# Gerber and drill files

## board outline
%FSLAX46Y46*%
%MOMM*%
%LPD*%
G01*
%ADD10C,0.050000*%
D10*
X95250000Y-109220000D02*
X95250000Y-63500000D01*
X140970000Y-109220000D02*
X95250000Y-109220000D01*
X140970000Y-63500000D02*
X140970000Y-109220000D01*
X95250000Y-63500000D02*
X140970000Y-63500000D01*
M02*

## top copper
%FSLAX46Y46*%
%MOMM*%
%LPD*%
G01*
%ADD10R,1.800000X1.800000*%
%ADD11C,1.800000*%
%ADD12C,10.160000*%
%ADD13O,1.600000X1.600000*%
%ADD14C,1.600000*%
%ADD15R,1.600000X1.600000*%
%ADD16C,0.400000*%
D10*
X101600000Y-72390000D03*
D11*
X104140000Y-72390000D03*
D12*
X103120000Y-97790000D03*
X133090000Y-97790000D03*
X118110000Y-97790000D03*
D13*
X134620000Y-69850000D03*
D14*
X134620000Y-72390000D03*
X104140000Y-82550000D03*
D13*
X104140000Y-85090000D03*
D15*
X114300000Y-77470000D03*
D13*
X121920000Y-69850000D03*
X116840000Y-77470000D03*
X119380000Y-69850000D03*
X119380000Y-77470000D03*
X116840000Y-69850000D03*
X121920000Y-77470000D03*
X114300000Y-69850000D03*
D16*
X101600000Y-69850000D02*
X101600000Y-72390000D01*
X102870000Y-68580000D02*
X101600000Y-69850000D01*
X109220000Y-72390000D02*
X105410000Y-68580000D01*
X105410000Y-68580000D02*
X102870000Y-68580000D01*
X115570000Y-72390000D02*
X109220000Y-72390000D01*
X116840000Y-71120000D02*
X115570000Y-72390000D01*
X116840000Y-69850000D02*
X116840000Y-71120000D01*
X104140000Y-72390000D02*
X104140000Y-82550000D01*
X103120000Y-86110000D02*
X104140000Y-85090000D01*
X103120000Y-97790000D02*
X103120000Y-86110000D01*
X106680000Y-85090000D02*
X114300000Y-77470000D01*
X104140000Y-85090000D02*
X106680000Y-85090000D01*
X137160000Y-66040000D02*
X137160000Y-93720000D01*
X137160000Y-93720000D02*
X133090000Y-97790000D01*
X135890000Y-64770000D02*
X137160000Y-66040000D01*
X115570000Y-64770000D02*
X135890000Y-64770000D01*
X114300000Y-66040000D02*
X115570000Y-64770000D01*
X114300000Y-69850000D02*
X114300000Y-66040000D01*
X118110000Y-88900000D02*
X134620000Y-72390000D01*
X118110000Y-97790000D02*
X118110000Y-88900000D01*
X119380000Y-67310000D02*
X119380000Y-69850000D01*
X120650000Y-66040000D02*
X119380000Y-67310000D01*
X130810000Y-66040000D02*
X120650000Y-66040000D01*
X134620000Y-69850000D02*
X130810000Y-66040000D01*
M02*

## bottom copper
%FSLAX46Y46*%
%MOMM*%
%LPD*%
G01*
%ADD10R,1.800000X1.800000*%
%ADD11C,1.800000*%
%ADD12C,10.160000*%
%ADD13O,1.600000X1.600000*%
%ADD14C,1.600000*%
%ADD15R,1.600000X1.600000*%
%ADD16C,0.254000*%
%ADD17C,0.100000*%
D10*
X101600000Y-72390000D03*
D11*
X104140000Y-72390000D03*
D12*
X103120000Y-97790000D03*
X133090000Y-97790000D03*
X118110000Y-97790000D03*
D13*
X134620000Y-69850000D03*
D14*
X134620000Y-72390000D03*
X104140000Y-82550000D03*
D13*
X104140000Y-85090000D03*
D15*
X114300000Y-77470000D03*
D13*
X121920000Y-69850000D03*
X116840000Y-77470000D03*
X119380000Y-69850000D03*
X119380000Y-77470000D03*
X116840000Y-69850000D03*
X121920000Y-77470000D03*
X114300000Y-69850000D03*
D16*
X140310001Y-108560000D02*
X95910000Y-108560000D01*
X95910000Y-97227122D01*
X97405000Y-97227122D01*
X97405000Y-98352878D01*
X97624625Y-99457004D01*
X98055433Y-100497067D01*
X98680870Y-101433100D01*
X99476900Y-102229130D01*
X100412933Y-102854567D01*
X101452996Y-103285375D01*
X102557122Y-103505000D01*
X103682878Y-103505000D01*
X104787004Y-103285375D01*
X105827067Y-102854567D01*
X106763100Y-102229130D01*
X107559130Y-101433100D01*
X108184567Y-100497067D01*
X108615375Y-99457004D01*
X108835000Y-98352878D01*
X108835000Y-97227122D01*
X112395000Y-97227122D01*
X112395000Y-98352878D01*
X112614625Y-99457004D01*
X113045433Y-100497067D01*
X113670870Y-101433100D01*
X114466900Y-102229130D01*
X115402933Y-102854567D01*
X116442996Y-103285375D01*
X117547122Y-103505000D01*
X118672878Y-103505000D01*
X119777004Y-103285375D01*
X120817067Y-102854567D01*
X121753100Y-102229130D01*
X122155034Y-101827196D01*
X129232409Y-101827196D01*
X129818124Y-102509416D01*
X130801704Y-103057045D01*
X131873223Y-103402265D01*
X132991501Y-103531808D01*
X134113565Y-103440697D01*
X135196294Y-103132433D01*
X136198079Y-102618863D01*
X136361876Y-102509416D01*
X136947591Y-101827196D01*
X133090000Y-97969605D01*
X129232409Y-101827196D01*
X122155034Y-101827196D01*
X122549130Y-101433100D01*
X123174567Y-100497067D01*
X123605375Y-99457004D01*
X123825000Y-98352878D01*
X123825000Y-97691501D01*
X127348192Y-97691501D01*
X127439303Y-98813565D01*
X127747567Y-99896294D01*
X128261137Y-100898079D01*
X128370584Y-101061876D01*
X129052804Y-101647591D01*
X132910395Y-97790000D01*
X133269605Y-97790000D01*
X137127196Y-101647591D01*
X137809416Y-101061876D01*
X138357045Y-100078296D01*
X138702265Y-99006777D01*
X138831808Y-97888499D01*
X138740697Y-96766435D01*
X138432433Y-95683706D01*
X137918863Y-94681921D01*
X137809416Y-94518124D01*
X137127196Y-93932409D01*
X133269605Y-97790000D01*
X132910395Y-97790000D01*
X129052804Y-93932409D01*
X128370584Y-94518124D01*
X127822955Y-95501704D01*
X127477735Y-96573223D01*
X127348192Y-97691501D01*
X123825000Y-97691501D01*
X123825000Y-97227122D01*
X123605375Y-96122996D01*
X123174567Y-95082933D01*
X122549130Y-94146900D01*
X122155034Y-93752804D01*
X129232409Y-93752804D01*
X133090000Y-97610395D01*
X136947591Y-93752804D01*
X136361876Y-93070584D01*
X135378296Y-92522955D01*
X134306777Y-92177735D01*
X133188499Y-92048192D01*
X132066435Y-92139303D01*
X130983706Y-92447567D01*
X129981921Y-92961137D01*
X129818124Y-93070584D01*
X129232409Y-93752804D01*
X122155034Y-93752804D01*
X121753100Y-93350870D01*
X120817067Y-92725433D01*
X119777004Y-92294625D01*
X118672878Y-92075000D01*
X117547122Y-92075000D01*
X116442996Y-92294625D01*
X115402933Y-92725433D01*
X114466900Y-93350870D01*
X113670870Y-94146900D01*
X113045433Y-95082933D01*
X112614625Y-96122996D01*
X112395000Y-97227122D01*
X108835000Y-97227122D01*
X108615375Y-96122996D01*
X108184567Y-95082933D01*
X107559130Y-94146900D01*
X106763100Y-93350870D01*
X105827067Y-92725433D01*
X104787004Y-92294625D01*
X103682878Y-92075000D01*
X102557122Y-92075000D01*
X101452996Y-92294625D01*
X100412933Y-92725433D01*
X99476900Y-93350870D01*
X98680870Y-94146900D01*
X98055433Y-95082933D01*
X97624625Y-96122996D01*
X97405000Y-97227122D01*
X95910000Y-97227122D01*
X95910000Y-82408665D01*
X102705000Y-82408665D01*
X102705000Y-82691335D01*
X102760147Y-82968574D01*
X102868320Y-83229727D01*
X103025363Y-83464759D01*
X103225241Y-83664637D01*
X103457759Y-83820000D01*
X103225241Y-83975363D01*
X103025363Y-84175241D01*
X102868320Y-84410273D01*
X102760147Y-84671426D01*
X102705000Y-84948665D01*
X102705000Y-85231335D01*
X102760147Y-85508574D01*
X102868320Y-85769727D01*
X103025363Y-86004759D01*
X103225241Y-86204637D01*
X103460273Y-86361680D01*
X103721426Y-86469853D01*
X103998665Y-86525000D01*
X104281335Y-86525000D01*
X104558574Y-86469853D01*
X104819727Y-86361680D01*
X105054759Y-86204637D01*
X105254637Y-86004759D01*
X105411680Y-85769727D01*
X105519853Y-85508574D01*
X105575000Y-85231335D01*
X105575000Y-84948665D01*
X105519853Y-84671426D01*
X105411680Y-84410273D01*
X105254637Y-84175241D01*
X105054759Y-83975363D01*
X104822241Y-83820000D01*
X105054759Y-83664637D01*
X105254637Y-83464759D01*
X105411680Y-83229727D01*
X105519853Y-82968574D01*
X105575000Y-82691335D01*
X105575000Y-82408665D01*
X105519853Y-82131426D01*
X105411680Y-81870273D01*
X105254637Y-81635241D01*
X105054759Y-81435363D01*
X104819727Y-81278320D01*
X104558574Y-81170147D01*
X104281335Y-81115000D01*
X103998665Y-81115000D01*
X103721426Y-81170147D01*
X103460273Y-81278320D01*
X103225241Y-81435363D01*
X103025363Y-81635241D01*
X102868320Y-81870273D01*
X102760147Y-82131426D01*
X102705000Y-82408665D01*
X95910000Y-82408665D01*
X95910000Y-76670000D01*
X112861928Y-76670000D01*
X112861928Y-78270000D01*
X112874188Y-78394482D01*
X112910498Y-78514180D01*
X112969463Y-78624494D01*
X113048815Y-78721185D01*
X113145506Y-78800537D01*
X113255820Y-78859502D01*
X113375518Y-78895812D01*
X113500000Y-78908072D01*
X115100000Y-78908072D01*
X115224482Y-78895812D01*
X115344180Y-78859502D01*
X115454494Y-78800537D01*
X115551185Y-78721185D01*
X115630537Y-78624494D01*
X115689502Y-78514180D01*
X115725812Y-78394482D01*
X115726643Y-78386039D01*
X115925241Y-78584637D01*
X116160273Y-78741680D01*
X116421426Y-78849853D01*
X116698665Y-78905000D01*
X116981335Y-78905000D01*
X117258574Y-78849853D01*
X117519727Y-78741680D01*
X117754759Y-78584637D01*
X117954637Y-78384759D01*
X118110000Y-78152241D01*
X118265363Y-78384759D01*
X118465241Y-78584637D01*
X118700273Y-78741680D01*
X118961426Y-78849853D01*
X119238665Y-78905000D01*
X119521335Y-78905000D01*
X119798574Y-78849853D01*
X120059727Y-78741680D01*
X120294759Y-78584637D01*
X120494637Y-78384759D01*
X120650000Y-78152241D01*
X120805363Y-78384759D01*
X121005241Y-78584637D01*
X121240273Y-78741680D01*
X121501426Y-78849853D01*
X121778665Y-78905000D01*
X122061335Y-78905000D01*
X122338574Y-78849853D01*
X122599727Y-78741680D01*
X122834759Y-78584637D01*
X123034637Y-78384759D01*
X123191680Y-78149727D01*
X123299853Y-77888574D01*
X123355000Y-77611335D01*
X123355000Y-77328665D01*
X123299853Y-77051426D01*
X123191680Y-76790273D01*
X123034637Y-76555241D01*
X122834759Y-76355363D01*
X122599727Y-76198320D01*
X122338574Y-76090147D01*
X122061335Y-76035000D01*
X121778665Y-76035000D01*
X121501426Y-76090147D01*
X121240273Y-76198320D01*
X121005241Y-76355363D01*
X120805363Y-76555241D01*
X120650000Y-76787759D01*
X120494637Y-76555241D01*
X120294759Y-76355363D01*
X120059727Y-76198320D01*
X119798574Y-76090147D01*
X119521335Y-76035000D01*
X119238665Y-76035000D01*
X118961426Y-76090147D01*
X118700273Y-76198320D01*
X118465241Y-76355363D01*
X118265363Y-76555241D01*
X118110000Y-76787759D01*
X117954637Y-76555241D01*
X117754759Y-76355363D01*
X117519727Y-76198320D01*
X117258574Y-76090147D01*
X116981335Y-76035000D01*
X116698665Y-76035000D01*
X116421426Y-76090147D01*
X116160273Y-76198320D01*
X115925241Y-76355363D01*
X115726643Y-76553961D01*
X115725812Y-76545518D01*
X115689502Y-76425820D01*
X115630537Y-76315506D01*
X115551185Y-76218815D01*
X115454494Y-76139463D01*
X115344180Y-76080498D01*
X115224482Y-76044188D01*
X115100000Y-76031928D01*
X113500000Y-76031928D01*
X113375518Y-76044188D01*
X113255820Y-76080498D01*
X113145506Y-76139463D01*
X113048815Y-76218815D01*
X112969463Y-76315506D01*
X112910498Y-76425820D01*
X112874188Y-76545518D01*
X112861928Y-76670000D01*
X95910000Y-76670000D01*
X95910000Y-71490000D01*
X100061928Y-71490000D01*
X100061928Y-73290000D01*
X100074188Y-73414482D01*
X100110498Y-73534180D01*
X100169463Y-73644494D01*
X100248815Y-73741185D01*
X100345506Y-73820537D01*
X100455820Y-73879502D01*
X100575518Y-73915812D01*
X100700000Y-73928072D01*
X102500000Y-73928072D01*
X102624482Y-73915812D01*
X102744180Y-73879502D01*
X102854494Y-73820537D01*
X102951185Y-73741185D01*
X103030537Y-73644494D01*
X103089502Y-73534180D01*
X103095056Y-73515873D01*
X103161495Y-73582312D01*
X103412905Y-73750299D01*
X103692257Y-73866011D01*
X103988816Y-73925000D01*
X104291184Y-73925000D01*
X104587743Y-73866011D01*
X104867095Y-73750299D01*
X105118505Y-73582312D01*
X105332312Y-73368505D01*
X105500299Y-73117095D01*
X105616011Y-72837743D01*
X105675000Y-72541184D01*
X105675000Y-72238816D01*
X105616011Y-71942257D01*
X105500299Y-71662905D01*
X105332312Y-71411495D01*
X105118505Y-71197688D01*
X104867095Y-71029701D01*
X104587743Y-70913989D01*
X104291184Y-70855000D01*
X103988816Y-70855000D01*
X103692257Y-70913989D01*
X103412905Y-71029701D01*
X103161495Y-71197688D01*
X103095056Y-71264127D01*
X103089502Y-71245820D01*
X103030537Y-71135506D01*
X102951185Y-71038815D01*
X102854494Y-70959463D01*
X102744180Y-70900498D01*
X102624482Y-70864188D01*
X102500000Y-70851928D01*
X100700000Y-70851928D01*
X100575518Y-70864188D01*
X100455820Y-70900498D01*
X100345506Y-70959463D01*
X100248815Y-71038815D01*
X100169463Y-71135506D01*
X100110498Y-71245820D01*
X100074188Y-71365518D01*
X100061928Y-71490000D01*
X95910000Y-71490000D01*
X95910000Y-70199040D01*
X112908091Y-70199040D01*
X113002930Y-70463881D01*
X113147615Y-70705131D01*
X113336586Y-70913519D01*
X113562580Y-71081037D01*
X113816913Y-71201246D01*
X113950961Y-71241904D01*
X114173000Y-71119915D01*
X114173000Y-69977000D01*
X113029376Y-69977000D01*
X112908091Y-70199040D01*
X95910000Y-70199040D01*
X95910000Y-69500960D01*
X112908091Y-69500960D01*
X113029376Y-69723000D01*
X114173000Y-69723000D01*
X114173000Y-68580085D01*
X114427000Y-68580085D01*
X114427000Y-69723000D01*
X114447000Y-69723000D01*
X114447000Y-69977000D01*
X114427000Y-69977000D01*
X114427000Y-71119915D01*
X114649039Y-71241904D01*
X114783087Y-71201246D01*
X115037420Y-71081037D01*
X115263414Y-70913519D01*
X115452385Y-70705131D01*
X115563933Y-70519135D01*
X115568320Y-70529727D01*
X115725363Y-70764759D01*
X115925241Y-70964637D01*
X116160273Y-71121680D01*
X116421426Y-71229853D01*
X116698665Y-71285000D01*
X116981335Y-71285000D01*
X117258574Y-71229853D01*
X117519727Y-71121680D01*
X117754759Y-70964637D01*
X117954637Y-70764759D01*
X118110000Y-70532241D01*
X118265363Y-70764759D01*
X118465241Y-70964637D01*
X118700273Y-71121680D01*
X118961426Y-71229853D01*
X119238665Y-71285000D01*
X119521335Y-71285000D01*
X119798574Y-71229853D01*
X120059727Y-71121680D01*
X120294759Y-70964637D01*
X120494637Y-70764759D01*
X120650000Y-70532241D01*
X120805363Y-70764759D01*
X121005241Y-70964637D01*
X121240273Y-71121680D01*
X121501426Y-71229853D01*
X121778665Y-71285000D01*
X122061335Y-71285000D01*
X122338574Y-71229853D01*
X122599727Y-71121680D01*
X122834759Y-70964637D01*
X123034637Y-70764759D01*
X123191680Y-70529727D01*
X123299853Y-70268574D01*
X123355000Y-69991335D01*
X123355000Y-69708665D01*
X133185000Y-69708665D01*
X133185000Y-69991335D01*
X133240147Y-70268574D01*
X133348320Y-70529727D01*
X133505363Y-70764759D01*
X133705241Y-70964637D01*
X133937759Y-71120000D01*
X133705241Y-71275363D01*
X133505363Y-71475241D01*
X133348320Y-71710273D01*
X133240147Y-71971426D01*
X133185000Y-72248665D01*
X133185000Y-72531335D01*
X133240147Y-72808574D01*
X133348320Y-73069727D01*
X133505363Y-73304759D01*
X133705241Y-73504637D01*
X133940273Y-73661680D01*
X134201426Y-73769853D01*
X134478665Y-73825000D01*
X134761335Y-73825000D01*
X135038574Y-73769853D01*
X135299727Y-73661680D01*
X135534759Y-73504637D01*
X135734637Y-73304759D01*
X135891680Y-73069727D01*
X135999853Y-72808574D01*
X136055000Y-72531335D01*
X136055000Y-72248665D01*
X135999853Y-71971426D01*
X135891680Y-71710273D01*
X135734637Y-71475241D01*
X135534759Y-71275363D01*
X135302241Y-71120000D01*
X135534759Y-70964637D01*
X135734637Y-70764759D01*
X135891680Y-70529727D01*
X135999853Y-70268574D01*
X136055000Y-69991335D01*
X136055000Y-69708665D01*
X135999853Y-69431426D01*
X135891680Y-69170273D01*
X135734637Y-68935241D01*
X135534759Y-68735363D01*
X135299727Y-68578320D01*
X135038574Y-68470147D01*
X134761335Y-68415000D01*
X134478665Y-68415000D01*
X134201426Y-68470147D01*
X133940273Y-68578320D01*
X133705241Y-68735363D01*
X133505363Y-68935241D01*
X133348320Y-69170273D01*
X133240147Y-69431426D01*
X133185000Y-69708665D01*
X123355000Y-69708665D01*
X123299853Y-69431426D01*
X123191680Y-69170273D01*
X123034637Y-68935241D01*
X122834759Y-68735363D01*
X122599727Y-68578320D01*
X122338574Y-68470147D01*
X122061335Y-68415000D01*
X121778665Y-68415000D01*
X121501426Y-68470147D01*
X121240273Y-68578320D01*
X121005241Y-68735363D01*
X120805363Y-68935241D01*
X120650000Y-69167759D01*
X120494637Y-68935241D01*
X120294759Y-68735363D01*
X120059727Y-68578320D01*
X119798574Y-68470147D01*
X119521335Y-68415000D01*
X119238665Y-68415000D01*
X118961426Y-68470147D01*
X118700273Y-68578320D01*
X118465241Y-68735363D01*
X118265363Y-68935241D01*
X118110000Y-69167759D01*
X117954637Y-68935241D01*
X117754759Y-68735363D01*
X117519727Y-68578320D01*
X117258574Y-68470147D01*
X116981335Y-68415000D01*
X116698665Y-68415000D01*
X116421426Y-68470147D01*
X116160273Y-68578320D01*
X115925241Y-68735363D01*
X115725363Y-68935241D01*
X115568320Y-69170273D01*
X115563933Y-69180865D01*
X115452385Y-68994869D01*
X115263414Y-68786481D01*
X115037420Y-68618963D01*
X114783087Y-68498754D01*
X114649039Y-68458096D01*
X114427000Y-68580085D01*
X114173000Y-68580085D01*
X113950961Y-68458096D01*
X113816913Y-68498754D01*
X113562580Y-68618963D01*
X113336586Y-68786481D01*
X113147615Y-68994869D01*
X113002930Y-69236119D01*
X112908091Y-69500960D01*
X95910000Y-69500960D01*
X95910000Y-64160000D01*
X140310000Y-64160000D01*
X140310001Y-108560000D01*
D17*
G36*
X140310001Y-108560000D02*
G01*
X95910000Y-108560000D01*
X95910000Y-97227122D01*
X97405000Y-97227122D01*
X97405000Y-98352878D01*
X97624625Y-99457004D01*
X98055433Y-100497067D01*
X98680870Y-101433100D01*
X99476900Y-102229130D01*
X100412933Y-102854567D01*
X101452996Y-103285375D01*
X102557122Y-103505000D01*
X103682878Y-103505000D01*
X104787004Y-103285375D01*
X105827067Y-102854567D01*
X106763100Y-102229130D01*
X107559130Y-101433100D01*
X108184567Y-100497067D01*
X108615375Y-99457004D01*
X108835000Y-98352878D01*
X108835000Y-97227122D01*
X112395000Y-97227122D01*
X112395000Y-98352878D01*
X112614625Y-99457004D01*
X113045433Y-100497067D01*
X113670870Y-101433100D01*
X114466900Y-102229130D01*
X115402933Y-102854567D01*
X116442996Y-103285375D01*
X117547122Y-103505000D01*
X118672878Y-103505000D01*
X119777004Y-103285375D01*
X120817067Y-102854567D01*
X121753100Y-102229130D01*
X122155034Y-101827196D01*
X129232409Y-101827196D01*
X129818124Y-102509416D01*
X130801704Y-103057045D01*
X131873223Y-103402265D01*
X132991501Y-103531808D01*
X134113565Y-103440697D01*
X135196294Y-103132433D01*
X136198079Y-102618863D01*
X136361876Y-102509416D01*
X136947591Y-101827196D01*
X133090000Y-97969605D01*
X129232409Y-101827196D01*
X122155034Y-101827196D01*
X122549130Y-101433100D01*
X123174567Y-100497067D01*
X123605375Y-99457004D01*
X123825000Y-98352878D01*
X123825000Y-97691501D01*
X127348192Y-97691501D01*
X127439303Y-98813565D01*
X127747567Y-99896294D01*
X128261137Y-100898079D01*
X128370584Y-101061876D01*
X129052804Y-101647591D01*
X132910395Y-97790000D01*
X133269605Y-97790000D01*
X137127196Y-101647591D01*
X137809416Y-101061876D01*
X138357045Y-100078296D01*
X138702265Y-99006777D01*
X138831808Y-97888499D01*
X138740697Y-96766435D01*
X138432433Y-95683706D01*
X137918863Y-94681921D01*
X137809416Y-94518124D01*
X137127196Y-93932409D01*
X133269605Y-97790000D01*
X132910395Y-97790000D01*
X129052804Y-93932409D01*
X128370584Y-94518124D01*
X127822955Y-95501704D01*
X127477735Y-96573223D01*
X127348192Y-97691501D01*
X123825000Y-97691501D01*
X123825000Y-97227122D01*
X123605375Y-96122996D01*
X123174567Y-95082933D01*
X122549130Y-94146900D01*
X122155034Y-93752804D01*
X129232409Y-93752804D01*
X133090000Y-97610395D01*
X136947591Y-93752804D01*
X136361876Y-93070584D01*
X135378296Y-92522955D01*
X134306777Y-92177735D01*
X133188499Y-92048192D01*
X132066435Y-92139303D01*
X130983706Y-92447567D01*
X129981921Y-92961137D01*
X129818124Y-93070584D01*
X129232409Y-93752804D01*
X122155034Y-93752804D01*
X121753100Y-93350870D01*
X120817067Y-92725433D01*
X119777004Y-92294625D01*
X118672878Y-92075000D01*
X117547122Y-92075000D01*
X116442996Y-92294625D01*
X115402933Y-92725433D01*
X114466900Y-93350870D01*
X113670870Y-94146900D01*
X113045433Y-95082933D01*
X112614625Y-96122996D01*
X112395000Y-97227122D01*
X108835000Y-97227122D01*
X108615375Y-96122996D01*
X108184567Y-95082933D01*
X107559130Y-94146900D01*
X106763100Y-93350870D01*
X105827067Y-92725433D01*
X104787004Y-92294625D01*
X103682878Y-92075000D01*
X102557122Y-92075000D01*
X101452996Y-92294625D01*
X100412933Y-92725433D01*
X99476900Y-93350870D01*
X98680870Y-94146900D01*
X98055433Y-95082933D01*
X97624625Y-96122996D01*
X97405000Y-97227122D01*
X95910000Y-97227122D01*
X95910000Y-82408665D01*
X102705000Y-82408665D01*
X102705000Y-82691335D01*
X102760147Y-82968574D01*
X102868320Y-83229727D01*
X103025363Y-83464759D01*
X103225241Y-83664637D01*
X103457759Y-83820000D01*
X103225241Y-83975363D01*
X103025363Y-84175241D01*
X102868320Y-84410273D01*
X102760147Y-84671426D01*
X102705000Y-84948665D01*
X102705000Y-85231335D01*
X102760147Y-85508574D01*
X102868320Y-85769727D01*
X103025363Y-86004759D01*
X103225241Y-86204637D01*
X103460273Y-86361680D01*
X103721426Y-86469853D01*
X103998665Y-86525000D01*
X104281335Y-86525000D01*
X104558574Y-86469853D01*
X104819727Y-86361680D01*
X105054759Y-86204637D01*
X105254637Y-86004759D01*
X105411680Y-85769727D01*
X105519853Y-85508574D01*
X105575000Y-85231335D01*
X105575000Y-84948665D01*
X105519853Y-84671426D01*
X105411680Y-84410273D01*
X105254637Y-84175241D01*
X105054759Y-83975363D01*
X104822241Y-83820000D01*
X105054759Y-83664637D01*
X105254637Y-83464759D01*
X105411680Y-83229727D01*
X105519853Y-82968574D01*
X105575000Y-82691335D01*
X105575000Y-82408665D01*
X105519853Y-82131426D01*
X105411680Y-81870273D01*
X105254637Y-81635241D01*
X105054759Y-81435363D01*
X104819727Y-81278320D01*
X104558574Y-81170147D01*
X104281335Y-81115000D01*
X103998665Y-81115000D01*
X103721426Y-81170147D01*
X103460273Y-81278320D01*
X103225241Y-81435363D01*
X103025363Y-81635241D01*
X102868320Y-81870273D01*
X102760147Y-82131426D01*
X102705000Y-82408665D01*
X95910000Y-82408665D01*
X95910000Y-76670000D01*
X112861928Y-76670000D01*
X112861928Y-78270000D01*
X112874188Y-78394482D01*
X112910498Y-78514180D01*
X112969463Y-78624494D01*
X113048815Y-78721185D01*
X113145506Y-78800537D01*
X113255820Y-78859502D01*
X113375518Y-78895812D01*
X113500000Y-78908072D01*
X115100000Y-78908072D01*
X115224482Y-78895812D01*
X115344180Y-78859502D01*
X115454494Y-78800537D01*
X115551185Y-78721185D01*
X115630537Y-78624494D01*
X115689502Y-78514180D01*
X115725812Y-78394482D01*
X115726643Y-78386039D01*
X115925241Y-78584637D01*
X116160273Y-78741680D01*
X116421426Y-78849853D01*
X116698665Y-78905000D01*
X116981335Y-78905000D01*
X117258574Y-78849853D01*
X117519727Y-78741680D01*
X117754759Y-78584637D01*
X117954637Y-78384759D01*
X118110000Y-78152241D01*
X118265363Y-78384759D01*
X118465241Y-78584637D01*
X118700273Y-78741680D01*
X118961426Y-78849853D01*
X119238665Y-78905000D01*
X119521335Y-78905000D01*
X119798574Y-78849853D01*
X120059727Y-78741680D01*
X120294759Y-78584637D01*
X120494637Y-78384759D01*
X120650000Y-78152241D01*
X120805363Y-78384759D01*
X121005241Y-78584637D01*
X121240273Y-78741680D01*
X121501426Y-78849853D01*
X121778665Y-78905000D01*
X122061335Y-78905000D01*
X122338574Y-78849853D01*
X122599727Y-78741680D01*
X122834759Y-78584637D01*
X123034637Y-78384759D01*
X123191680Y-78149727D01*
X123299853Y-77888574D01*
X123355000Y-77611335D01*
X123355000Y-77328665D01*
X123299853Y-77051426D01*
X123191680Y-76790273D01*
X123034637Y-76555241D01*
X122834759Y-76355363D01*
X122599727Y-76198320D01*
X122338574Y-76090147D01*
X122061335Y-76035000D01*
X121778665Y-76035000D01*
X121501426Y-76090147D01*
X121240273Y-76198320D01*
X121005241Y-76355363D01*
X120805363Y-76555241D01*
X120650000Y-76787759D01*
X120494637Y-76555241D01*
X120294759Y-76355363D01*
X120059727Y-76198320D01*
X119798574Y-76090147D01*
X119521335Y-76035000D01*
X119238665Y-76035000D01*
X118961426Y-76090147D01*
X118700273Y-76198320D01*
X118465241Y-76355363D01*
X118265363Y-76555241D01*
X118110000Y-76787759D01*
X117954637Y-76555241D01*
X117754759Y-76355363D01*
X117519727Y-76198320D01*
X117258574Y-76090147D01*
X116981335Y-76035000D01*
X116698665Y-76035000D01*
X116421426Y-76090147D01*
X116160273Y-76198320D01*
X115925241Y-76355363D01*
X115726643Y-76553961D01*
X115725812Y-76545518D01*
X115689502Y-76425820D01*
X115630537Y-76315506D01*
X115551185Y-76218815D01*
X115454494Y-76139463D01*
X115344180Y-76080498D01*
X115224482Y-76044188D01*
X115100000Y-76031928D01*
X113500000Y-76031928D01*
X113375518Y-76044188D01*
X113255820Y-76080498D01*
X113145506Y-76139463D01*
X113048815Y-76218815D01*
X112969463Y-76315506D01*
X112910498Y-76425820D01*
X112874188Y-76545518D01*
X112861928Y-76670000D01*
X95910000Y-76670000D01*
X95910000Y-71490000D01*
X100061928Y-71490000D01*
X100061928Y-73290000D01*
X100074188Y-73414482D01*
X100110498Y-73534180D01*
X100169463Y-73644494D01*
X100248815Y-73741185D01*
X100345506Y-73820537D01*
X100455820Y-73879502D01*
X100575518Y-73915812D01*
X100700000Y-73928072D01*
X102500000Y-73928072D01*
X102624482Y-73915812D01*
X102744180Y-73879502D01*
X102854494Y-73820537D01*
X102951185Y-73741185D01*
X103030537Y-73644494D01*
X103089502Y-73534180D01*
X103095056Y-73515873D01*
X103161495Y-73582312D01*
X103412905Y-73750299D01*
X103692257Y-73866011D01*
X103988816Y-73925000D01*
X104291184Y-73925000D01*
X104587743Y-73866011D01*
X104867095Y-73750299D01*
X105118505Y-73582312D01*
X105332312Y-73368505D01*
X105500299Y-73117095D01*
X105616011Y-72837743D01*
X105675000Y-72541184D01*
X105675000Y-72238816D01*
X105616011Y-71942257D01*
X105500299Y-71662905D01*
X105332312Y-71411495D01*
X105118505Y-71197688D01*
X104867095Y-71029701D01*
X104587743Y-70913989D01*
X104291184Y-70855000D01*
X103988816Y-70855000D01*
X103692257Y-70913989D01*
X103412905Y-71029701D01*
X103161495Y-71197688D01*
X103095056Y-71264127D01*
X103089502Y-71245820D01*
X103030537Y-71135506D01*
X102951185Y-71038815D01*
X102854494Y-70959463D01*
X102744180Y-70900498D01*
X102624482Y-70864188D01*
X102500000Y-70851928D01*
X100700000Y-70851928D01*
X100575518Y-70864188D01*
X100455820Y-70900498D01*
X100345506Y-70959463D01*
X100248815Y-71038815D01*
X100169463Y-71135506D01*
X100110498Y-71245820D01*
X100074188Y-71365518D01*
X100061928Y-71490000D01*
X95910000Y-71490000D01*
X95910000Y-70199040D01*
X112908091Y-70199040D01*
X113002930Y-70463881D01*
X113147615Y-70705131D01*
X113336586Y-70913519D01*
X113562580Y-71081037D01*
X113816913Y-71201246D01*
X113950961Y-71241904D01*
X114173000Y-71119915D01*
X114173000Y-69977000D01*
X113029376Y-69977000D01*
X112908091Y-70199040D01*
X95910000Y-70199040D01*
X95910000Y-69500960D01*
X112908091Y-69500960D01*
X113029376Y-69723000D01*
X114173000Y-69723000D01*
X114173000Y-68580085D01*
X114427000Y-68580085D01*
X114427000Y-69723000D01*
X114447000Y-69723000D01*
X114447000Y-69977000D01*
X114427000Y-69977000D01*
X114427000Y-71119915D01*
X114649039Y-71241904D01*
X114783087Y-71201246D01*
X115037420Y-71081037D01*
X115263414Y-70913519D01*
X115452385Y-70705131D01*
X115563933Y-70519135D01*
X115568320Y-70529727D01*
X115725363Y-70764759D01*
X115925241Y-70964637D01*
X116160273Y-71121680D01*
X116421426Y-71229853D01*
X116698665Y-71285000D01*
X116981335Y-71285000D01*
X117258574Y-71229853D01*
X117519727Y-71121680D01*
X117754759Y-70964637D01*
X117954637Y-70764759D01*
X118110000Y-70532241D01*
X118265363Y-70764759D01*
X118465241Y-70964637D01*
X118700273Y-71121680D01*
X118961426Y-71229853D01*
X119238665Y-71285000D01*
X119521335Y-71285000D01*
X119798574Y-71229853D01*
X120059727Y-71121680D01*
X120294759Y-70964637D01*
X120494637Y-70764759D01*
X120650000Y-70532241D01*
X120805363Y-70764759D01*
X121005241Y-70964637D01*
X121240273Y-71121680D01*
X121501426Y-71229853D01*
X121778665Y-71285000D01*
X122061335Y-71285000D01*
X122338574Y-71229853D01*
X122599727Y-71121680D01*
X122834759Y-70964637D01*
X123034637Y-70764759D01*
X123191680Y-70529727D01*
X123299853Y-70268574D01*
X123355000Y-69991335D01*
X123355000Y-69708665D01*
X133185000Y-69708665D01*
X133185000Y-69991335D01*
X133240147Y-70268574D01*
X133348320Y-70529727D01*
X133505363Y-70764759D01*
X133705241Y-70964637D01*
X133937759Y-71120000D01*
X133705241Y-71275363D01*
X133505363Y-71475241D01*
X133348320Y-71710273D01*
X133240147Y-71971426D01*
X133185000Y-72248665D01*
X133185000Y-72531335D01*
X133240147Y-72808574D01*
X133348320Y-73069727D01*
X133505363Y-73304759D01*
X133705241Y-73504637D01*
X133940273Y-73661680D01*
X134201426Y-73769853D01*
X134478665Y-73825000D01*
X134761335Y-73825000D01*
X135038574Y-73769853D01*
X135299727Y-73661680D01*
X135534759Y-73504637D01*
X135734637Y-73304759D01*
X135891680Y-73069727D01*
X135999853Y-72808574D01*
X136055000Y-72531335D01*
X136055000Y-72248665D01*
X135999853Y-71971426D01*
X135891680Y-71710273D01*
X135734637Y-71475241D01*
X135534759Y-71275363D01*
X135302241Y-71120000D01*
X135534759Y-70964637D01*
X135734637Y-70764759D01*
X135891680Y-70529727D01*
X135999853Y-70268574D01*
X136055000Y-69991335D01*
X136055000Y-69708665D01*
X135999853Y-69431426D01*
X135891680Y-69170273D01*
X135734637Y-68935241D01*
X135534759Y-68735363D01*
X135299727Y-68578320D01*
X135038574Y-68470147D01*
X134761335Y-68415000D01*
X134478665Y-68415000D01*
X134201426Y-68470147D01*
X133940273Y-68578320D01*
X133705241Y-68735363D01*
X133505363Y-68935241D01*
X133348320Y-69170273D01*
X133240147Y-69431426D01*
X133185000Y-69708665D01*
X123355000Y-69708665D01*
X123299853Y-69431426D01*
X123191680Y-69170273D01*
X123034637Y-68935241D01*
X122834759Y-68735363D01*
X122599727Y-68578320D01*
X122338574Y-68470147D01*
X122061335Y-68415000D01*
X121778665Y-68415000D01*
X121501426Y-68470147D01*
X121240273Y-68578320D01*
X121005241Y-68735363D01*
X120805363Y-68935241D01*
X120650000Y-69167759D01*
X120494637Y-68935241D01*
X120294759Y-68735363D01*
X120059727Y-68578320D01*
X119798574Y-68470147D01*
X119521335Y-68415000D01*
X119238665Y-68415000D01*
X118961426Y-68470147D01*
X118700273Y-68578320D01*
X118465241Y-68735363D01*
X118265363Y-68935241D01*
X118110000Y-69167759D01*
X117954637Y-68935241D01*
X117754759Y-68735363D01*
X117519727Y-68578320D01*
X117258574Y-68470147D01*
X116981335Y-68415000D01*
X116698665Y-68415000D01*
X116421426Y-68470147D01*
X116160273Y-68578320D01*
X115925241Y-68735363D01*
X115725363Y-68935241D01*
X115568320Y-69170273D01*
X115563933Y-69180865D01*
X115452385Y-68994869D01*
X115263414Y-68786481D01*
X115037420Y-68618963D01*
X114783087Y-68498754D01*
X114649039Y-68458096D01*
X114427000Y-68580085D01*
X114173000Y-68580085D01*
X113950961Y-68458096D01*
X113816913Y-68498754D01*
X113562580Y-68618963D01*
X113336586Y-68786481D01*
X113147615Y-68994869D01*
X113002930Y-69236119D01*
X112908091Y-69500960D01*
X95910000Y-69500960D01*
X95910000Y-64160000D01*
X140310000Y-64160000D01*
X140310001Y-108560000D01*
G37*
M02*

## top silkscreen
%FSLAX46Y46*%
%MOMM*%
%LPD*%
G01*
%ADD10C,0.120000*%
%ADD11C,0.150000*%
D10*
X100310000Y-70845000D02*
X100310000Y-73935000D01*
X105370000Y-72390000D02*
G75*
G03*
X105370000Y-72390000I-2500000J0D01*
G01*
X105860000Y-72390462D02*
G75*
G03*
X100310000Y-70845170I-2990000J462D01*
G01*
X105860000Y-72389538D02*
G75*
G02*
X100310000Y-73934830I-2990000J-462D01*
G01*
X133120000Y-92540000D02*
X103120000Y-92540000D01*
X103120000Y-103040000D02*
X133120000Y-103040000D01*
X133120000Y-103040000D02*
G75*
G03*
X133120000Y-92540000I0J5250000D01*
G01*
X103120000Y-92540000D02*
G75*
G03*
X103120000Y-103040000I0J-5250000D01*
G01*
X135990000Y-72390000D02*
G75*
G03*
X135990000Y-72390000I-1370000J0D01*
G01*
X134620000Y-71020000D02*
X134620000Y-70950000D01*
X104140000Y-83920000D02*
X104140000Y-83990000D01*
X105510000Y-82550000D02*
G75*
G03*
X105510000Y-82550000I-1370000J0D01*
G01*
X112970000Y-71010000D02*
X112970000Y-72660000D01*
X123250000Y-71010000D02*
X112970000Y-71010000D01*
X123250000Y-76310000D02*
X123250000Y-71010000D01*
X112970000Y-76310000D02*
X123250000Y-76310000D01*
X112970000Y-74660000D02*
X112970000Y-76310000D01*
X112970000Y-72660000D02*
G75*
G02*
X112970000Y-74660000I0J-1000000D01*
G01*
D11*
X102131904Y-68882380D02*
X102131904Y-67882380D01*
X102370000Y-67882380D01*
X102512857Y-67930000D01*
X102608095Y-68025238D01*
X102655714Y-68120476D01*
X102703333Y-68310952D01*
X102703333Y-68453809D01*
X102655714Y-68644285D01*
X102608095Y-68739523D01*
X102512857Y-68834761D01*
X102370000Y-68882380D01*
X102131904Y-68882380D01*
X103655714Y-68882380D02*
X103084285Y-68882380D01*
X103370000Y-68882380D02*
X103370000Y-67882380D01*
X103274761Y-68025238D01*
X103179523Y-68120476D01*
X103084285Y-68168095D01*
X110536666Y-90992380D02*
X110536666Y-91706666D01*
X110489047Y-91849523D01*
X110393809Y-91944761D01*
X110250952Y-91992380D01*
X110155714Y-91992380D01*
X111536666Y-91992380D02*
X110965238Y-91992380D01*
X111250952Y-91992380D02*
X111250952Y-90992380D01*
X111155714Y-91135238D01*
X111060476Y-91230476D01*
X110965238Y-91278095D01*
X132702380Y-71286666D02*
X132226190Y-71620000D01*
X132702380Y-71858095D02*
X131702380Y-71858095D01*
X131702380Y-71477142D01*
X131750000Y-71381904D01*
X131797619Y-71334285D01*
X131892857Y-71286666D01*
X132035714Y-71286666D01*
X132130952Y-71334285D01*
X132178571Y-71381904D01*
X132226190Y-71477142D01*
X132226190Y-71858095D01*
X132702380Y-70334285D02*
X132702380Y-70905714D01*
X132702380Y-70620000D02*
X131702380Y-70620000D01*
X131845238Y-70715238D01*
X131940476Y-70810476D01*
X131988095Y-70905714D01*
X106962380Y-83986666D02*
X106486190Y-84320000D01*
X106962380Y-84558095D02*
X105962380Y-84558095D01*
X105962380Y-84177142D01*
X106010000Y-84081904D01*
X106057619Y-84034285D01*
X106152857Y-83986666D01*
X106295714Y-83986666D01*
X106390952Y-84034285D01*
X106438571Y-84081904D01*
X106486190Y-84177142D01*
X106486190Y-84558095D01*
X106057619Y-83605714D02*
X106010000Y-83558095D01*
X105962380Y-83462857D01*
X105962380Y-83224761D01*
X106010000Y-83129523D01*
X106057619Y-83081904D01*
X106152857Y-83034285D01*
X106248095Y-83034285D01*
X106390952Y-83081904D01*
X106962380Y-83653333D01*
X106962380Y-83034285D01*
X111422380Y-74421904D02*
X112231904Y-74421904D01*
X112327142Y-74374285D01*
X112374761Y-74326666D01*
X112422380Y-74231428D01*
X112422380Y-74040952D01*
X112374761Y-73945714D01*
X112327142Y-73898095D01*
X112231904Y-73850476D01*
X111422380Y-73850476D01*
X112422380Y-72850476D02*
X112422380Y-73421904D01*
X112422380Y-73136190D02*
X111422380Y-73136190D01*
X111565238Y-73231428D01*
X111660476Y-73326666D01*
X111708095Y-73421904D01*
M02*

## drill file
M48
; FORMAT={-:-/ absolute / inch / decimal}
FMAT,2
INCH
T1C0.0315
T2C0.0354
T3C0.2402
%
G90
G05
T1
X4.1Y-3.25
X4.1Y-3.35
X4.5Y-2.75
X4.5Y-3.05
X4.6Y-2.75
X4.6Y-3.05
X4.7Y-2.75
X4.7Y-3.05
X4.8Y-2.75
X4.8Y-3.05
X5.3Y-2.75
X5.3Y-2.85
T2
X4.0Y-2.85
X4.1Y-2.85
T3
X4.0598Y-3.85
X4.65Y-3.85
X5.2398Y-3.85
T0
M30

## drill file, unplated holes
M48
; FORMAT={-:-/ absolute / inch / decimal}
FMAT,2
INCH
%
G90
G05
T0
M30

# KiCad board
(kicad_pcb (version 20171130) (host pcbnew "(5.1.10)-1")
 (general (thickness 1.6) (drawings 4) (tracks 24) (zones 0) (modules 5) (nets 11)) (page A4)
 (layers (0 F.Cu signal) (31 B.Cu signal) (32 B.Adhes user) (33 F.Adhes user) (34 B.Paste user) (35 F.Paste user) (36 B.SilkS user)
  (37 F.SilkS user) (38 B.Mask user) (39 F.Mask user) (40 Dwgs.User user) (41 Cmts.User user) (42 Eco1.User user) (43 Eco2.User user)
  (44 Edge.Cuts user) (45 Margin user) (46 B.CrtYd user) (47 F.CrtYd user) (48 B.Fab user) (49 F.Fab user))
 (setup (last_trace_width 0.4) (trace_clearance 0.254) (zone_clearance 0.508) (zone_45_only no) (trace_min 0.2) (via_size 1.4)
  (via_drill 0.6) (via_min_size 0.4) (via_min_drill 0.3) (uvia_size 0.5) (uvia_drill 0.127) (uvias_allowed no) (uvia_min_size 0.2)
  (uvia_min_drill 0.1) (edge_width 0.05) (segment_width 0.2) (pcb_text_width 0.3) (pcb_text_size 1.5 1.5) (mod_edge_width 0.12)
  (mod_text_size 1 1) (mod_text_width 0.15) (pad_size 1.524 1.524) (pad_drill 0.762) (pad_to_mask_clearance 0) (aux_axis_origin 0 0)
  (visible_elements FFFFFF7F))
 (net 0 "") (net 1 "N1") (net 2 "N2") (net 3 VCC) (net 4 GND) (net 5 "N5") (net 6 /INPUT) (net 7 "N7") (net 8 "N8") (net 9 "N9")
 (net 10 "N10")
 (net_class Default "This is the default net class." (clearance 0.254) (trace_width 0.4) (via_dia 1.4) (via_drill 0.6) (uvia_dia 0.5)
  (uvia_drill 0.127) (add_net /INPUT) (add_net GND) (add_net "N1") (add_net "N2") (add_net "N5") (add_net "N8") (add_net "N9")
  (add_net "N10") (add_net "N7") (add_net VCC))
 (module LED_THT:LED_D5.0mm (layer F.Cu) (at 101.6 72.39)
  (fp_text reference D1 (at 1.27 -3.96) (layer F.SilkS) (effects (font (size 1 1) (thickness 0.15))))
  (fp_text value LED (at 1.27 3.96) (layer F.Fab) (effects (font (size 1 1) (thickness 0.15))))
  (fp_line (start -1.29 -1.545) (end -1.29 1.545) (layer F.SilkS) (width 0.12))
  (fp_circle (center 1.27 0) (end 3.77 0) (layer F.SilkS) (width 0.12))
  (fp_arc (start 1.27 0) (end -1.29 -1.54483) (angle 148.9) (layer F.SilkS) (width 0.12))
  (fp_arc (start 1.27 0) (end -1.29 1.54483) (angle -148.9) (layer F.SilkS) (width 0.12))
  (pad 1 thru_hole rect (at 0 0) (size 1.8 1.8) (drill 0.9) (layers *.Cu *.Mask) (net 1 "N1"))
  (pad 2 thru_hole circle (at 2.54 0) (size 1.8 1.8) (drill 0.9) (layers *.Cu *.Mask) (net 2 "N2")))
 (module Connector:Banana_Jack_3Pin (layer F.Cu) (at 103.12 97.79)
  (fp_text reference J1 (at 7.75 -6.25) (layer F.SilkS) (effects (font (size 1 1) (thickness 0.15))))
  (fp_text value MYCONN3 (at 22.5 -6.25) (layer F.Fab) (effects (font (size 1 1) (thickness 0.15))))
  (fp_line (start 30 -5.25) (end 0 -5.25) (layer F.SilkS) (width 0.12))
  (fp_line (start 0 5.25) (end 30 5.25) (layer F.SilkS) (width 0.12))
  (fp_arc (start 30 0) (end 30 -5.25) (angle 180) (layer F.SilkS) (width 0.12))
  (fp_arc (start 0 0) (end 0 5.25) (angle 180) (layer F.SilkS) (width 0.12))
  (pad 1 thru_hole circle (at 0 0) (size 10.16 10.16) (drill 6.1) (layers *.Cu *.Mask) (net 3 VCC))
  (pad 3 thru_hole circle (at 29.97 0) (size 10.16 10.16) (drill 6.1) (layers *.Cu *.Mask) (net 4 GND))
  (pad 2 thru_hole circle (at 14.99 0) (size 10.16 10.16) (drill 6.1) (layers *.Cu *.Mask) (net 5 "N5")))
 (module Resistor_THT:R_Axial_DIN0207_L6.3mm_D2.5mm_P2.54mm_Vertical (layer F.Cu) (at 134.62 72.39 90)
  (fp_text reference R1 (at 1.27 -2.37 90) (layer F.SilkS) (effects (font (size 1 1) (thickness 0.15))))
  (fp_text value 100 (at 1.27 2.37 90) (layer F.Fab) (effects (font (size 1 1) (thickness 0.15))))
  (fp_circle (center 0 0) (end 1.37 0) (layer F.SilkS) (width 0.12))
  (fp_line (start 1.37 0) (end 1.44 0) (layer F.SilkS) (width 0.12))
  (pad 2 thru_hole oval (at 2.54 0 90) (size 1.6 1.6) (drill 0.8) (layers *.Cu *.Mask) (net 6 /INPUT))
  (pad 1 thru_hole circle (at 0 0 90) (size 1.6 1.6) (drill 0.8) (layers *.Cu *.Mask) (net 5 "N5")))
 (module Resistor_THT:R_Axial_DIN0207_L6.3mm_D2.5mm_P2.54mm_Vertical (layer F.Cu) (at 104.14 82.55 270)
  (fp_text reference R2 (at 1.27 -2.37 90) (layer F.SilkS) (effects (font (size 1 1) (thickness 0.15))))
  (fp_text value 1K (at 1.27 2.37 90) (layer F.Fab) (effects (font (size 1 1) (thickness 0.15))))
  (fp_line (start 1.37 0) (end 1.44 0) (layer F.SilkS) (width 0.12))
  (fp_circle (center 0 0) (end 1.37 0) (layer F.SilkS) (width 0.12))
  (pad 1 thru_hole circle (at 0 0 270) (size 1.6 1.6) (drill 0.8) (layers *.Cu *.Mask) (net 2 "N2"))
  (pad 2 thru_hole oval (at 2.54 0 270) (size 1.6 1.6) (drill 0.8) (layers *.Cu *.Mask) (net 3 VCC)))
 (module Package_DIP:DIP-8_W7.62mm (layer F.Cu) (at 114.3 77.47 90)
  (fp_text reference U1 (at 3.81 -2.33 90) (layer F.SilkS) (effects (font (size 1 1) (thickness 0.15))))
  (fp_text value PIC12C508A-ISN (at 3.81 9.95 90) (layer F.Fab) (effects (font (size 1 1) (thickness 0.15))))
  (fp_line (start 6.46 -1.33) (end 4.81 -1.33) (layer F.SilkS) (width 0.12))
  (fp_line (start 6.46 8.95) (end 6.46 -1.33) (layer F.SilkS) (width 0.12))
  (fp_line (start 1.16 8.95) (end 6.46 8.95) (layer F.SilkS) (width 0.12))
  (fp_line (start 1.16 -1.33) (end 1.16 8.95) (layer F.SilkS) (width 0.12))
  (fp_line (start 2.81 -1.33) (end 1.16 -1.33) (layer F.SilkS) (width 0.12))
  (fp_arc (start 3.81 -1.33) (end 2.81 -1.33) (angle -180) (layer F.SilkS) (width 0.12))
  (pad 1 thru_hole rect (at 0 0 90) (size 1.6 1.6) (drill 0.8) (layers *.Cu *.Mask) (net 3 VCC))
  (pad 5 thru_hole oval (at 7.62 7.62 90) (size 1.6 1.6) (drill 0.8) (layers *.Cu *.Mask) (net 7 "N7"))
  (pad 2 thru_hole oval (at 0 2.54 90) (size 1.6 1.6) (drill 0.8) (layers *.Cu *.Mask) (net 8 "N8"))
  (pad 6 thru_hole oval (at 7.62 5.08 90) (size 1.6 1.6) (drill 0.8) (layers *.Cu *.Mask) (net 6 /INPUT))
  (pad 3 thru_hole oval (at 0 5.08 90) (size 1.6 1.6) (drill 0.8) (layers *.Cu *.Mask) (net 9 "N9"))
  (pad 7 thru_hole oval (at 7.62 2.54 90) (size 1.6 1.6) (drill 0.8) (layers *.Cu *.Mask) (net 1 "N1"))
  (pad 4 thru_hole oval (at 0 7.62 90) (size 1.6 1.6) (drill 0.8) (layers *.Cu *.Mask) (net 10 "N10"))
  (pad 8 thru_hole oval (at 7.62 0 90) (size 1.6 1.6) (drill 0.8) (layers *.Cu *.Mask) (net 4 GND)))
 (gr_line (start 95.25 109.22) (end 95.25 63.5) (layer Edge.Cuts) (width 0.05))
 (gr_line (start 140.97 109.22) (end 95.25 109.22) (layer Edge.Cuts) (width 0.05))
 (gr_line (start 140.97 63.5) (end 140.97 109.22) (layer Edge.Cuts) (width 0.05))
 (gr_line (start 95.25 63.5) (end 140.97 63.5) (layer Edge.Cuts) (width 0.05))
 (segment (start 101.6 69.85) (end 101.6 72.39) (width 0.4) (layer F.Cu) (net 1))
 (segment (start 102.87 68.58) (end 101.6 69.85) (width 0.4) (layer F.Cu) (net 1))
 (segment (start 109.22 72.39) (end 105.41 68.58) (width 0.4) (layer F.Cu) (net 1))
 (segment (start 105.41 68.58) (end 102.87 68.58) (width 0.4) (layer F.Cu) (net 1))
 (segment (start 115.57 72.39) (end 109.22 72.39) (width 0.4) (layer F.Cu) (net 1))
 (segment (start 116.84 71.12) (end 115.57 72.39) (width 0.4) (layer F.Cu) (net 1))
 (segment (start 116.84 69.85) (end 116.84 71.12) (width 0.4) (layer F.Cu) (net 1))
 (segment (start 104.14 72.39) (end 104.14 82.55) (width 0.4) (layer F.Cu) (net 2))
 (segment (start 103.12 86.11) (end 104.14 85.09) (width 0.4) (layer F.Cu) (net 3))
 (segment (start 103.12 97.79) (end 103.12 86.11) (width 0.4) (layer F.Cu) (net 3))
 (segment (start 106.68 85.09) (end 114.3 77.47) (width 0.4) (layer F.Cu) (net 3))
 (segment (start 104.14 85.09) (end 106.68 85.09) (width 0.4) (layer F.Cu) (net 3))
 (segment (start 137.16 66.04) (end 137.16 93.72) (width 0.4) (layer F.Cu) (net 4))
 (segment (start 137.16 93.72) (end 133.09 97.79) (width 0.4) (layer F.Cu) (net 4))
 (segment (start 135.89 64.77) (end 137.16 66.04) (width 0.4) (layer F.Cu) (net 4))
 (segment (start 115.57 64.77) (end 135.89 64.77) (width 0.4) (layer F.Cu) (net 4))
 (segment (start 114.3 66.04) (end 115.57 64.77) (width 0.4) (layer F.Cu) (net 4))
 (segment (start 114.3 69.85) (end 114.3 66.04) (width 0.4) (layer F.Cu) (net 4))
 (segment (start 118.11 88.9) (end 134.62 72.39) (width 0.4) (layer F.Cu) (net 5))
 (segment (start 118.11 97.79) (end 118.11 88.9) (width 0.4) (layer F.Cu) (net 5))
 (segment (start 119.38 67.31) (end 119.38 69.85) (width 0.4) (layer F.Cu) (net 6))
 (segment (start 120.65 66.04) (end 119.38 67.31) (width 0.4) (layer F.Cu) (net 6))
 (segment (start 130.81 66.04) (end 120.65 66.04) (width 0.4) (layer F.Cu) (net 6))
 (segment (start 134.62 69.85) (end 130.81 66.04) (width 0.4) (layer F.Cu) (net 6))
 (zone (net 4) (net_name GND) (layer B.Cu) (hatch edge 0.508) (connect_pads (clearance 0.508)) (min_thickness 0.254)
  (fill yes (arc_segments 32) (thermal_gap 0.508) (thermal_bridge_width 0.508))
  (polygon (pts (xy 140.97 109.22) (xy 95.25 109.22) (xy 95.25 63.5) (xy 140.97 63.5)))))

